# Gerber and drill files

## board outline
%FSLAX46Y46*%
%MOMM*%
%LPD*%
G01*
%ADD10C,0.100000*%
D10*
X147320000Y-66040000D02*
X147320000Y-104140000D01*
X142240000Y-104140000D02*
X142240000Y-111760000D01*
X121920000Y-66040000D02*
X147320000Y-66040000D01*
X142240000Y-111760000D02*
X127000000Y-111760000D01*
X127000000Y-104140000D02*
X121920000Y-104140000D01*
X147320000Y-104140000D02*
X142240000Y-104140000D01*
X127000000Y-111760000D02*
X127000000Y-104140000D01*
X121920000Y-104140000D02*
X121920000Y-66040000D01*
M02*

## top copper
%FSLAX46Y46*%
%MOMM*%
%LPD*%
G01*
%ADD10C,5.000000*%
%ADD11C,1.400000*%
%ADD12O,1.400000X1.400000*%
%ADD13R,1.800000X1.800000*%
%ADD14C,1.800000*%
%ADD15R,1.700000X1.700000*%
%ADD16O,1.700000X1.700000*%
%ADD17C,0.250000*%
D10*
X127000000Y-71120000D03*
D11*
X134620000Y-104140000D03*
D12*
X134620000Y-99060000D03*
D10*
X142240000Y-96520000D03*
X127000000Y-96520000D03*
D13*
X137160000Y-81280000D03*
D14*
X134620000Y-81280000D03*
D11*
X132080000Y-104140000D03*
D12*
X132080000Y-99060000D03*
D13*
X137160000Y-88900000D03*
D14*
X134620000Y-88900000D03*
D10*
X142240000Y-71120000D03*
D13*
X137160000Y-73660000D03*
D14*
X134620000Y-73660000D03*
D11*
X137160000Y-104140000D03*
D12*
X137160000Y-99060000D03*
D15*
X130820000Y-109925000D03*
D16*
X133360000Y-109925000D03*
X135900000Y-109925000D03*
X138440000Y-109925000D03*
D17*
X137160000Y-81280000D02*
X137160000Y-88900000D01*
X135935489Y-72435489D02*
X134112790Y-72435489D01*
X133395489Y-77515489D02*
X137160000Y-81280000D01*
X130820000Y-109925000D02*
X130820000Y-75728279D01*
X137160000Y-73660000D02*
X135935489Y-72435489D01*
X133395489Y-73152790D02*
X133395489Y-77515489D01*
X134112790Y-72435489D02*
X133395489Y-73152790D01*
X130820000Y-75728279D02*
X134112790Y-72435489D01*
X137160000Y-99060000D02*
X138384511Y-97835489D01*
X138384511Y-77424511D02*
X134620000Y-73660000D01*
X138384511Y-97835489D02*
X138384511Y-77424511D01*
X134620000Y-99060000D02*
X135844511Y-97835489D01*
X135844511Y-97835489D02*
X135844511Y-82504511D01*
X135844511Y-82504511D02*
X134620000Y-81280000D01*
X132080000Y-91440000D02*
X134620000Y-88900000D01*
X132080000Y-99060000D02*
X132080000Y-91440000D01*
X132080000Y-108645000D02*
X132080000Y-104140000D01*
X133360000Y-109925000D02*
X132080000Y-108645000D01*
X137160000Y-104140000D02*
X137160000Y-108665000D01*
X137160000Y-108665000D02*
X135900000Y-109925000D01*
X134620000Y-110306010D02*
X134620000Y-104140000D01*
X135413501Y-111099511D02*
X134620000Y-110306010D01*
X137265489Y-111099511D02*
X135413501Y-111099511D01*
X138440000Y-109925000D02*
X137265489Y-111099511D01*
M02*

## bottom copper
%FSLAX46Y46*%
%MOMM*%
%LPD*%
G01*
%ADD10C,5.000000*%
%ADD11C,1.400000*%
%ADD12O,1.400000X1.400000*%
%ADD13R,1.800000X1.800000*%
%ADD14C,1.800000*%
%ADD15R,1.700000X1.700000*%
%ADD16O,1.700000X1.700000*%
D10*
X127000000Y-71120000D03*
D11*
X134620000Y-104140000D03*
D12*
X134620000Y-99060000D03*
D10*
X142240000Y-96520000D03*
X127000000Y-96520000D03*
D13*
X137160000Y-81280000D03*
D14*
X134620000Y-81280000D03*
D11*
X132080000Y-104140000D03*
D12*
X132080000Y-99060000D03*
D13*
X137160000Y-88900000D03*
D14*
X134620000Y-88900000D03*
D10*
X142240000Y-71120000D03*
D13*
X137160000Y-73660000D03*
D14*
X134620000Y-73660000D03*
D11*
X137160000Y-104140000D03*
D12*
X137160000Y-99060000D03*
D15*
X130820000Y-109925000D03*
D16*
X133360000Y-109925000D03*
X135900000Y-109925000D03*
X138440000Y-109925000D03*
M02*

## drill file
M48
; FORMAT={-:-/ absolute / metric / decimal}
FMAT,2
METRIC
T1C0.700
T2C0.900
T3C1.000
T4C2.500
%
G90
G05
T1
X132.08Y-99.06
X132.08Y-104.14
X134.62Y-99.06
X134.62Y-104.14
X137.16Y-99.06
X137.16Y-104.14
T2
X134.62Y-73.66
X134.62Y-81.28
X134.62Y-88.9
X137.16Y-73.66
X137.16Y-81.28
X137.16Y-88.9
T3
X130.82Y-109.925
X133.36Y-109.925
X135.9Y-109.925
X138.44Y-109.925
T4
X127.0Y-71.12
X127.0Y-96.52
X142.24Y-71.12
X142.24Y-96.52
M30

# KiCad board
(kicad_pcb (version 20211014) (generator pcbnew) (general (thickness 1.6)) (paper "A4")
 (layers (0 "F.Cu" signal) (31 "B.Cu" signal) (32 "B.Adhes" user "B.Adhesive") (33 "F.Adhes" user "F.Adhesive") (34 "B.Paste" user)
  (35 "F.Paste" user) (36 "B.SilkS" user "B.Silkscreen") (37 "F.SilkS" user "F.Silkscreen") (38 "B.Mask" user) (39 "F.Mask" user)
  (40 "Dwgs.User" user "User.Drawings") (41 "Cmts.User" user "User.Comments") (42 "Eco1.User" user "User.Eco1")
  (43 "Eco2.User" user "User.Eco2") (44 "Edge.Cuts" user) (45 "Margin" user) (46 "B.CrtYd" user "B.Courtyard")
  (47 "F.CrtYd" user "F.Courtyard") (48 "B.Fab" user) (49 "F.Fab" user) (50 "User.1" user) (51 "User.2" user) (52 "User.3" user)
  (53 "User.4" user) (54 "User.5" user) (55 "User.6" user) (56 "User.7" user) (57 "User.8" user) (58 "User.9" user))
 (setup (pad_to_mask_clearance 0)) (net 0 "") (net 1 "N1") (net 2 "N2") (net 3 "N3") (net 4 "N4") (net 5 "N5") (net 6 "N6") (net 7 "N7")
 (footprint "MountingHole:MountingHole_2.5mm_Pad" (layer "F.Cu") (at 127 71.12)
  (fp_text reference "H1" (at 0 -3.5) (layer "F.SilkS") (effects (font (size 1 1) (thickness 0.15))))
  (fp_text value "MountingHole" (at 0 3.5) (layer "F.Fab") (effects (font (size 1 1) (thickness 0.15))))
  (pad "1" thru_hole circle (at 0 0) (size 5 5) (drill 2.5) (layers *.Cu *.Mask)))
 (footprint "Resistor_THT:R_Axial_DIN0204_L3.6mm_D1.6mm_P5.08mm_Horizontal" (layer "F.Cu") (at 134.62 104.14 90)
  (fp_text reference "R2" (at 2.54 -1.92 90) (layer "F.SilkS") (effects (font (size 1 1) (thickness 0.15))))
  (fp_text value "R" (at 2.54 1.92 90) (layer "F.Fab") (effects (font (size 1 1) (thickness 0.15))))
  (pad "1" thru_hole circle (at 0 0 90) (size 1.4 1.4) (drill 0.7) (layers *.Cu *.Mask) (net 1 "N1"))
  (pad "2" thru_hole oval (at 5.08 0 90) (size 1.4 1.4) (drill 0.7) (layers *.Cu *.Mask) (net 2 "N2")))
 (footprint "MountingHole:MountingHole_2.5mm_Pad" (layer "F.Cu") (at 142.24 96.52)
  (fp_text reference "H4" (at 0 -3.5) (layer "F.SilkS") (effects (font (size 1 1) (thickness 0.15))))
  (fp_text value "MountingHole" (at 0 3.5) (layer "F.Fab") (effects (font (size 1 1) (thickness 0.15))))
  (pad "1" thru_hole circle (at 0 0) (size 5 5) (drill 2.5) (layers *.Cu *.Mask)))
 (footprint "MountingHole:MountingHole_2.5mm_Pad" (layer "F.Cu") (at 127 96.52)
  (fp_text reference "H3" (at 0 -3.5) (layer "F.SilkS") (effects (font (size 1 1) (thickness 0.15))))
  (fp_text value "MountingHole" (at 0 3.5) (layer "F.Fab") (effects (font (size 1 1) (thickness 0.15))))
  (pad "1" thru_hole circle (at 0 0) (size 5 5) (drill 2.5) (layers *.Cu *.Mask)))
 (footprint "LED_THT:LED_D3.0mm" (layer "F.Cu") (at 137.16 81.28 180)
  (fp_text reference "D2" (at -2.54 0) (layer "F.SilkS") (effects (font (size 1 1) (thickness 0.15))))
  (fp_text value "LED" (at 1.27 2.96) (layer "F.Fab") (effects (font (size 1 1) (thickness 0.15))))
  (pad "1" thru_hole rect (at 0 0 180) (size 1.8 1.8) (drill 0.9) (layers *.Cu *.Mask) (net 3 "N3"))
  (pad "2" thru_hole circle (at 2.54 0 180) (size 1.8 1.8) (drill 0.9) (layers *.Cu *.Mask) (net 2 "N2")))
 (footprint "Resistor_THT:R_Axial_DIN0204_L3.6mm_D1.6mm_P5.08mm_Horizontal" (layer "F.Cu") (at 132.08 104.14 90)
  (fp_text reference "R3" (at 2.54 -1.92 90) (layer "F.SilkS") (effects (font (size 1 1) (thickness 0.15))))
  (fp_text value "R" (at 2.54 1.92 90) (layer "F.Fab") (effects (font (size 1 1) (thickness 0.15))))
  (pad "1" thru_hole circle (at 0 0 90) (size 1.4 1.4) (drill 0.7) (layers *.Cu *.Mask) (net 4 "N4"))
  (pad "2" thru_hole oval (at 5.08 0 90) (size 1.4 1.4) (drill 0.7) (layers *.Cu *.Mask) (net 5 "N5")))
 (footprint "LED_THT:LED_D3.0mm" (layer "F.Cu") (at 137.16 88.9 180)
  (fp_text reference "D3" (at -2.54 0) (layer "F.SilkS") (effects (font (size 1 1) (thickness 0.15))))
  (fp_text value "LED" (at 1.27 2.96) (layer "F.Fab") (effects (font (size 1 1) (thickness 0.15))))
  (pad "1" thru_hole rect (at 0 0 180) (size 1.8 1.8) (drill 0.9) (layers *.Cu *.Mask) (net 3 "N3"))
  (pad "2" thru_hole circle (at 2.54 0 180) (size 1.8 1.8) (drill 0.9) (layers *.Cu *.Mask) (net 5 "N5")))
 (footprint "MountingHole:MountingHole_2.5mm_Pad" (layer "F.Cu") (at 142.24 71.12)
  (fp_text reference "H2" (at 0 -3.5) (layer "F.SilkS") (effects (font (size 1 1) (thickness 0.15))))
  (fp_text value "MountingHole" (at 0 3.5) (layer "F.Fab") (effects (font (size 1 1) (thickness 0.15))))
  (pad "1" thru_hole circle (at 0 0) (size 5 5) (drill 2.5) (layers *.Cu *.Mask)))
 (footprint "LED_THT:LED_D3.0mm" (layer "F.Cu") (at 137.16 73.66 180)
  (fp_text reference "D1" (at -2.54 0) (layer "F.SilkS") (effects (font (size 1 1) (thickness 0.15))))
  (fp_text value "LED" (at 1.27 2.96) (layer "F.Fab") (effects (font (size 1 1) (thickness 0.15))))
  (pad "1" thru_hole rect (at 0 0 180) (size 1.8 1.8) (drill 0.9) (layers *.Cu *.Mask) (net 3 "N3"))
  (pad "2" thru_hole circle (at 2.54 0 180) (size 1.8 1.8) (drill 0.9) (layers *.Cu *.Mask) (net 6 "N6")))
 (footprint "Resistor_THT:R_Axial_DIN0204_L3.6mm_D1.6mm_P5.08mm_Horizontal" (layer "F.Cu") (at 137.16 104.14 90)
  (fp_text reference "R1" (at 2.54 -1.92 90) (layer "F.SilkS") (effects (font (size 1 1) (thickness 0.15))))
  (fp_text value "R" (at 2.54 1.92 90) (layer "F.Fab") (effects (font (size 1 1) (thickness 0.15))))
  (pad "1" thru_hole circle (at 0 0 90) (size 1.4 1.4) (drill 0.7) (layers *.Cu *.Mask) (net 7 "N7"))
  (pad "2" thru_hole oval (at 5.08 0 90) (size 1.4 1.4) (drill 0.7) (layers *.Cu *.Mask) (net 6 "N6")))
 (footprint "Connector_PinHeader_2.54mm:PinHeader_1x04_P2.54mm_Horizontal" (layer "B.Cu") (at 130.82 109.925 -90)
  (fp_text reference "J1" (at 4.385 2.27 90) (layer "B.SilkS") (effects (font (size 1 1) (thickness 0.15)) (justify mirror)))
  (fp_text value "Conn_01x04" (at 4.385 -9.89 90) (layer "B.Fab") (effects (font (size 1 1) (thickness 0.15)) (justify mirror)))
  (pad "1" thru_hole rect (at 0 0 270) (size 1.7 1.7) (drill 1) (layers *.Cu *.Mask) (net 3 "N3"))
  (pad "2" thru_hole oval (at 0 -2.54 270) (size 1.7 1.7) (drill 1) (layers *.Cu *.Mask) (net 4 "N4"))
  (pad "3" thru_hole oval (at 0 -5.08 270) (size 1.7 1.7) (drill 1) (layers *.Cu *.Mask) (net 7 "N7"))
  (pad "4" thru_hole oval (at 0 -7.62 270) (size 1.7 1.7) (drill 1) (layers *.Cu *.Mask) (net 1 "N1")))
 (gr_line (start 147.32 66.04) (end 147.32 104.14) (layer "Edge.Cuts") (width 0.1))
 (gr_line (start 142.24 104.14) (end 142.24 111.76) (layer "Edge.Cuts") (width 0.1))
 (gr_line (start 121.92 66.04) (end 147.32 66.04) (layer "Edge.Cuts") (width 0.1))
 (gr_line (start 142.24 111.76) (end 127 111.76) (layer "Edge.Cuts") (width 0.1))
 (gr_line (start 127 104.14) (end 121.92 104.14) (layer "Edge.Cuts") (width 0.1))
 (gr_line (start 147.32 104.14) (end 142.24 104.14) (layer "Edge.Cuts") (width 0.1))
 (gr_line (start 127 111.76) (end 127 104.14) (layer "Edge.Cuts") (width 0.1))
 (gr_line (start 121.92 104.14) (end 121.92 66.04) (layer "Edge.Cuts") (width 0.1))
 (segment (start 137.16 81.28) (end 137.16 88.9) (width 0.25) (layer "F.Cu") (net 3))
 (segment (start 135.935489 72.435489) (end 134.11279 72.435489) (width 0.25) (layer "F.Cu") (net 3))
 (segment (start 133.395489 77.515489) (end 137.16 81.28) (width 0.25) (layer "F.Cu") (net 3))
 (segment (start 130.82 109.925) (end 130.82 75.728279) (width 0.25) (layer "F.Cu") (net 3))
 (segment (start 137.16 73.66) (end 135.935489 72.435489) (width 0.25) (layer "F.Cu") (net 3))
 (segment (start 133.395489 73.15279) (end 133.395489 77.515489) (width 0.25) (layer "F.Cu") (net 3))
 (segment (start 134.11279 72.435489) (end 133.395489 73.15279) (width 0.25) (layer "F.Cu") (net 3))
 (segment (start 130.82 75.728279) (end 134.11279 72.435489) (width 0.25) (layer "F.Cu") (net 3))
 (segment (start 137.16 99.06) (end 138.384511 97.835489) (width 0.25) (layer "F.Cu") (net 6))
 (segment (start 138.384511 77.424511) (end 134.62 73.66) (width 0.25) (layer "F.Cu") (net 6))
 (segment (start 138.384511 97.835489) (end 138.384511 77.424511) (width 0.25) (layer "F.Cu") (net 6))
 (segment (start 134.62 99.06) (end 135.844511 97.835489) (width 0.25) (layer "F.Cu") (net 2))
 (segment (start 135.844511 97.835489) (end 135.844511 82.504511) (width 0.25) (layer "F.Cu") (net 2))
 (segment (start 135.844511 82.504511) (end 134.62 81.28) (width 0.25) (layer "F.Cu") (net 2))
 (segment (start 132.08 91.44) (end 134.62 88.9) (width 0.25) (layer "F.Cu") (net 5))
 (segment (start 132.08 99.06) (end 132.08 91.44) (width 0.25) (layer "F.Cu") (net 5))
 (segment (start 132.08 108.645) (end 132.08 104.14) (width 0.25) (layer "F.Cu") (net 4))
 (segment (start 133.36 109.925) (end 132.08 108.645) (width 0.25) (layer "F.Cu") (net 4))
 (segment (start 137.16 104.14) (end 137.16 108.665) (width 0.25) (layer "F.Cu") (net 7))
 (segment (start 137.16 108.665) (end 135.9 109.925) (width 0.25) (layer "F.Cu") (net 7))
 (segment (start 134.62 110.30601) (end 134.62 104.14) (width 0.25) (layer "F.Cu") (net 1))
 (segment (start 135.413501 111.099511) (end 134.62 110.30601) (width 0.25) (layer "F.Cu") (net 1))
 (segment (start 137.265489 111.099511) (end 135.413501 111.099511) (width 0.25) (layer "F.Cu") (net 1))
 (segment (start 138.44 109.925) (end 137.265489 111.099511) (width 0.25) (layer "F.Cu") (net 1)))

